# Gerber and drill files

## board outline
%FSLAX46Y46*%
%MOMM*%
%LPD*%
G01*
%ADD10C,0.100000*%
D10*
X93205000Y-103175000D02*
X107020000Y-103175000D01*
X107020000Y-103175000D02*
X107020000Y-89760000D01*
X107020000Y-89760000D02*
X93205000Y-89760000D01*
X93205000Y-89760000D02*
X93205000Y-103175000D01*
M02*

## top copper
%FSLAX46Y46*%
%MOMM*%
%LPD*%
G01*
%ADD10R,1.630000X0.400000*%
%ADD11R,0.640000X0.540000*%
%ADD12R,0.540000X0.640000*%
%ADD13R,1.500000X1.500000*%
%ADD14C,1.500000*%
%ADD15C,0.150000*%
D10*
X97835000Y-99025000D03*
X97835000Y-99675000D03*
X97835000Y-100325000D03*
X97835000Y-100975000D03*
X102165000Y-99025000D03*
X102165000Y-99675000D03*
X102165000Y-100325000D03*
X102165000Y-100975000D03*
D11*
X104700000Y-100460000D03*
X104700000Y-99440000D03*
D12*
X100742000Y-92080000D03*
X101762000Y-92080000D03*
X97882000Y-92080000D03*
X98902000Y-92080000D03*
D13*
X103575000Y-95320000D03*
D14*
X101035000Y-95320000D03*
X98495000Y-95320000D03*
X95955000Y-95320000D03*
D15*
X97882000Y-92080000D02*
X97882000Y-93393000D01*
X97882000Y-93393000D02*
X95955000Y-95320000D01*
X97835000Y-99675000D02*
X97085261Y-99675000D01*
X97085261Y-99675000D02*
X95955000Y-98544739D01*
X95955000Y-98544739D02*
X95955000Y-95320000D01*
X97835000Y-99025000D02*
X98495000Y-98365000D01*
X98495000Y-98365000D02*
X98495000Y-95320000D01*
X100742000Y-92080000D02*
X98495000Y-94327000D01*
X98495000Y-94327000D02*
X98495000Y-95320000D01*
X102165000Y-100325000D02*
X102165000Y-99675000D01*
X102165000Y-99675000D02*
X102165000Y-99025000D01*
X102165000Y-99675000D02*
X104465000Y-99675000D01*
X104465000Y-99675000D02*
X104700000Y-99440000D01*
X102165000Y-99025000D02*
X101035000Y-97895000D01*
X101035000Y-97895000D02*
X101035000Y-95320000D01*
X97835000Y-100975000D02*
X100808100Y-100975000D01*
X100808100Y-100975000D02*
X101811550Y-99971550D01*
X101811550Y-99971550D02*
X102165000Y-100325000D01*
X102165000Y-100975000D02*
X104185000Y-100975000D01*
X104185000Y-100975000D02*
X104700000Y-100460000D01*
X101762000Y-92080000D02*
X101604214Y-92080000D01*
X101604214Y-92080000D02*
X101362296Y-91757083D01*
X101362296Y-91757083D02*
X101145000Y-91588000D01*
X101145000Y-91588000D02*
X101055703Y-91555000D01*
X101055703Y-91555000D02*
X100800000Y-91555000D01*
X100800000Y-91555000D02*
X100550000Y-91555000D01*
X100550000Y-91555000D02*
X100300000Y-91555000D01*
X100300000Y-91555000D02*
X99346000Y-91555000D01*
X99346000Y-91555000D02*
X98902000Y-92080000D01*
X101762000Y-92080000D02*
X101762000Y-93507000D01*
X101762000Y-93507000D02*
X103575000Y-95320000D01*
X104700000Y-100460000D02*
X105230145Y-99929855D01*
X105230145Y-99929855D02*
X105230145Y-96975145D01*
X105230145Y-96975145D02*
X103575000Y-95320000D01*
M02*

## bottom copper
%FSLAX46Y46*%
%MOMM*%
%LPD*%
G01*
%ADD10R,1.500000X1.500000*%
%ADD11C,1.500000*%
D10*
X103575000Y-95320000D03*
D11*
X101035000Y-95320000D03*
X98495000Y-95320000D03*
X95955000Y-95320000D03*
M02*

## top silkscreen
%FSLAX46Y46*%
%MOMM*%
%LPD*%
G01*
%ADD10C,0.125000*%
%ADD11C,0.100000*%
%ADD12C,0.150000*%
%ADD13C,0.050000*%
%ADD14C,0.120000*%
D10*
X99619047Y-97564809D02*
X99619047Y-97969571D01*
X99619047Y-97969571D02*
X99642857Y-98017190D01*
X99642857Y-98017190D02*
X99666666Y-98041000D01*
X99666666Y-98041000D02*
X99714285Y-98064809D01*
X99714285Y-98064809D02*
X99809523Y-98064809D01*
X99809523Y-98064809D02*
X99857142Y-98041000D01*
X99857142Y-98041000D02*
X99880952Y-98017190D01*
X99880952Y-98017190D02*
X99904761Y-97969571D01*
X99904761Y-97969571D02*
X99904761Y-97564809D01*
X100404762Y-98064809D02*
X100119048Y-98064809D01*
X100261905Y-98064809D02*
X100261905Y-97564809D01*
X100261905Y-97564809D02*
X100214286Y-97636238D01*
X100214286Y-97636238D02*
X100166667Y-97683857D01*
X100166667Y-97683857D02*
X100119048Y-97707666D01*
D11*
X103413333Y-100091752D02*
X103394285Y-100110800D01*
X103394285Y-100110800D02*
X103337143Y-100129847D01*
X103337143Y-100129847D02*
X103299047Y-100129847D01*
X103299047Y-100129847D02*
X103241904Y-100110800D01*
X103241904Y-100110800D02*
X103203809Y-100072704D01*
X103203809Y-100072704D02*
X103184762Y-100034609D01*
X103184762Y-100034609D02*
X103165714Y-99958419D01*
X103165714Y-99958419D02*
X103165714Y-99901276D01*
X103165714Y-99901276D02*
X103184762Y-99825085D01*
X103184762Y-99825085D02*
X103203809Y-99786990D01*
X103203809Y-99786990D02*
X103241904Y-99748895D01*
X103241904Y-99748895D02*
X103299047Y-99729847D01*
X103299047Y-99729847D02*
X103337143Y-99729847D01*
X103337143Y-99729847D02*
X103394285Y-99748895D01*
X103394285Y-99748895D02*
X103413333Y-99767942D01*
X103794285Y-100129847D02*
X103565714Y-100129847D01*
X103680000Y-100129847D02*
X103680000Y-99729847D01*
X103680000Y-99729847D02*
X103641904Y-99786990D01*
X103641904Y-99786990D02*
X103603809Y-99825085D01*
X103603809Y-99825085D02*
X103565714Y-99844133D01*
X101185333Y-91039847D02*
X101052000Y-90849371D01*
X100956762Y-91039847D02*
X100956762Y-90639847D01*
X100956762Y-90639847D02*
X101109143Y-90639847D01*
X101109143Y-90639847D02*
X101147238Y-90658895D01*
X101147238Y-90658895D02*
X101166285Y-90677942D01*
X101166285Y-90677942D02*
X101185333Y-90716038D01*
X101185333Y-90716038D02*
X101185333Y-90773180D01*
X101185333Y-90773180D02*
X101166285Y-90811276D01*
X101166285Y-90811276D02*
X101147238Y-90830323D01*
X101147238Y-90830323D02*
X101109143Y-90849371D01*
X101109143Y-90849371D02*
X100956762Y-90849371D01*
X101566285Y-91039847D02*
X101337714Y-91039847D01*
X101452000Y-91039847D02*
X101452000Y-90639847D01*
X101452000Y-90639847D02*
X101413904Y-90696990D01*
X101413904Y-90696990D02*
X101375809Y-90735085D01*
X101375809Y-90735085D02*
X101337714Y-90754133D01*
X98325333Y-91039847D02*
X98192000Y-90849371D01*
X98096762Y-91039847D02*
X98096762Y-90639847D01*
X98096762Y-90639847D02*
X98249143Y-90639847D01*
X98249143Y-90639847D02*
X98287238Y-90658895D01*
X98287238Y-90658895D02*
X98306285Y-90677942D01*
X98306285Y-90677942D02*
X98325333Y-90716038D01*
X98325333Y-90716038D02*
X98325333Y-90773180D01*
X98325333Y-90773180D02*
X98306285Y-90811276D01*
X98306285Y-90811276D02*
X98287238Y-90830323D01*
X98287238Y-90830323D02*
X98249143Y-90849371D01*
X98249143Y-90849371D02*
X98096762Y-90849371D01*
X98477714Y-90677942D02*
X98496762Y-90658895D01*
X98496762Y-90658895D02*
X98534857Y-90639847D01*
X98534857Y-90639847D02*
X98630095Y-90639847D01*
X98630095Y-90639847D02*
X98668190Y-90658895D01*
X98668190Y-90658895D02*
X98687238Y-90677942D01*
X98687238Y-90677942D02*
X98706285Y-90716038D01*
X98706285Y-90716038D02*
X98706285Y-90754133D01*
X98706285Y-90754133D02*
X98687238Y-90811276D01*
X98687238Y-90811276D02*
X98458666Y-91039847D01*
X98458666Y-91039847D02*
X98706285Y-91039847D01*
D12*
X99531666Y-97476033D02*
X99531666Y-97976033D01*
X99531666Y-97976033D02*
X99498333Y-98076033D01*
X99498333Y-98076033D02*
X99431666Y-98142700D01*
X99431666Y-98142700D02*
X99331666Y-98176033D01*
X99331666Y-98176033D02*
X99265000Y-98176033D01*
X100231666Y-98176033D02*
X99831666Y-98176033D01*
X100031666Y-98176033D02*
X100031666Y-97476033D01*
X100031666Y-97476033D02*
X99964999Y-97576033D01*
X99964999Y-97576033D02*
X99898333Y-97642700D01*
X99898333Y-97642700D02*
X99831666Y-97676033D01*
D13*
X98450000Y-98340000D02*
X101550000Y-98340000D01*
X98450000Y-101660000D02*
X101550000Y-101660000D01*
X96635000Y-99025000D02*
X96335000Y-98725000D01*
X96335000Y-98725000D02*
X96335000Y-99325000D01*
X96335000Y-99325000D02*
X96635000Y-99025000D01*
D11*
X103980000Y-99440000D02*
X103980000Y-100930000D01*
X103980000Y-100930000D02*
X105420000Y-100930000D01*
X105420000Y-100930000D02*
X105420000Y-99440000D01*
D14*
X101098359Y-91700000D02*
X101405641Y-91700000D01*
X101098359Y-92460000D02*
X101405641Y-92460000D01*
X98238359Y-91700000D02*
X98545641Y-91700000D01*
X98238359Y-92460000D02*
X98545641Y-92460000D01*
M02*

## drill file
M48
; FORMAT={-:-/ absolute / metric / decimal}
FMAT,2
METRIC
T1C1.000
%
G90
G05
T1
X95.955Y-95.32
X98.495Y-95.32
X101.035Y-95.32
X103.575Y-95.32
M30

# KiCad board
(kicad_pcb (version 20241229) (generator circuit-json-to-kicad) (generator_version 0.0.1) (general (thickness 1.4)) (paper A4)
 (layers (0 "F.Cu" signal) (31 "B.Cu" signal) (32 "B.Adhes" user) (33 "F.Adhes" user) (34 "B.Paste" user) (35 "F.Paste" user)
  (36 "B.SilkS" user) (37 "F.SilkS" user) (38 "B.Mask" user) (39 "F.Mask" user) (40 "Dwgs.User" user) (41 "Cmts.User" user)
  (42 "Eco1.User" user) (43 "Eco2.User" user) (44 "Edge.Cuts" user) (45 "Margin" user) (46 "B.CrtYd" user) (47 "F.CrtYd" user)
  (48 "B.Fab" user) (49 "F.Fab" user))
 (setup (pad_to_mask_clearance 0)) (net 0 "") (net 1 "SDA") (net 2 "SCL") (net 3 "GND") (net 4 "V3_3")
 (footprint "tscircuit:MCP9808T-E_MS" (layer F.Cu) (at 100 100 0)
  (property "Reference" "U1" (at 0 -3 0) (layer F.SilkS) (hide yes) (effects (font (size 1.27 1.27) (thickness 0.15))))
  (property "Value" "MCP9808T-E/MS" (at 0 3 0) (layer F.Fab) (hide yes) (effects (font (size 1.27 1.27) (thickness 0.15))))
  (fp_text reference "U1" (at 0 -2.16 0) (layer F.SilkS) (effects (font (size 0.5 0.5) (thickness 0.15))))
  (fp_line (start -1.55 -1.66) (end 1.55 -1.66) (stroke (width 0.05) (type default)) (layer F.SilkS))
  (fp_line (start -1.55 1.66) (end 1.55 1.66) (stroke (width 0.05) (type default)) (layer F.SilkS))
  (fp_line (start -3.3649999999999998 -0.9750000000000001) (end -3.665 -1.2750000000000001) (stroke (width 0.05) (type default))
   (layer F.SilkS))
  (fp_line (start -3.665 -1.2750000000000001) (end -3.665 -0.675) (stroke (width 0.05) (type default)) (layer F.SilkS))
  (fp_line (start -3.665 -0.675) (end -3.3649999999999998 -0.9750000000000001) (stroke (width 0.05) (type default)) (layer F.SilkS))
  (pad "1" smd rect (at -2.165 -0.9750000000000001 0) (size 1.63 0.4) (layers F.Cu F.Paste F.Mask) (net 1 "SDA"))
  (pad "2" smd rect (at -2.165 -0.325 0) (size 1.63 0.4) (layers F.Cu F.Paste F.Mask) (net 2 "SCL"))
  (pad "3" smd rect (at -2.165 0.325 0) (size 1.63 0.4) (layers F.Cu F.Paste F.Mask))
  (pad "4" smd rect (at -2.165 0.9750000000000001 0) (size 1.63 0.4) (layers F.Cu F.Paste F.Mask) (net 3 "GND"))
  (pad "5" smd rect (at 2.165 -0.9750000000000001 0) (size 1.63 0.4) (layers F.Cu F.Paste F.Mask) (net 3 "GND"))
  (pad "6" smd rect (at 2.165 -0.325 0) (size 1.63 0.4) (layers F.Cu F.Paste F.Mask) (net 3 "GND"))
  (pad "7" smd rect (at 2.165 0.325 0) (size 1.63 0.4) (layers F.Cu F.Paste F.Mask) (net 3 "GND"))
  (pad "8" smd rect (at 2.165 0.9750000000000001 0) (size 1.63 0.4) (layers F.Cu F.Paste F.Mask) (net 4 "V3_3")))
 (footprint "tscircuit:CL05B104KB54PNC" (layer F.Cu) (at 104.7 99.95 90)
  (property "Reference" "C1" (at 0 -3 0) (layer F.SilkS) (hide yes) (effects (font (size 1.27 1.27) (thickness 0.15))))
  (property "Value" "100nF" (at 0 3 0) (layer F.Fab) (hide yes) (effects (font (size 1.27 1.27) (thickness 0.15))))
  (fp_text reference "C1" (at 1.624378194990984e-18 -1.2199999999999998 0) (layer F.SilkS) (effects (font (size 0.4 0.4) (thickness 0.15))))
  (fp_line (start 0.51 -0.7199999999999998) (end -0.98 -0.7200000000000001) (stroke (width 0.1) (type default)) (layer F.SilkS))
  (fp_line (start -0.98 -0.7200000000000001) (end -0.98 0.7199999999999999) (stroke (width 0.1) (type default)) (layer F.SilkS))
  (fp_line (start -0.98 0.7199999999999999) (end 0.51 0.7199999999999998) (stroke (width 0.1) (type default)) (layer F.SilkS))
  (pad "1" smd rect (at -0.51 0 0) (size 0.64 0.54) (layers F.Cu F.Paste F.Mask) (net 4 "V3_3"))
  (pad "2" smd rect (at 0.51 0 0) (size 0.64 0.54) (layers F.Cu F.Paste F.Mask) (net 3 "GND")))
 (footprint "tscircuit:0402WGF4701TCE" (layer F.Cu) (at 101.252 92.08 0)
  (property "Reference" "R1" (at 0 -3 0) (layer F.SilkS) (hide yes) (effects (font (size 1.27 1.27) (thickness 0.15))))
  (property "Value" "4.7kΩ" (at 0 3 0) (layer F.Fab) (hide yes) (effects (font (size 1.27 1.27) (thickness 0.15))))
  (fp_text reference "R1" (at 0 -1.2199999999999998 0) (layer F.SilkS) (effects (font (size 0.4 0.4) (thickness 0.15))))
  (fp_line (start -0.15364099999999992 -0.3799999999999999) (end 0.15364099999999992 -0.3799999999999999)
   (stroke (width 0.12) (type default)) (layer F.SilkS))
  (fp_line (start -0.15364099999999992 0.3799999999999999) (end 0.15364099999999992 0.3799999999999999) (stroke (width 0.12) (type default))
   (layer F.SilkS))
  (pad "1" smd rect (at -0.51 0 0) (size 0.54 0.64) (layers F.Cu F.Paste F.Mask) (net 1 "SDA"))
  (pad "2" smd rect (at 0.51 0 0) (size 0.54 0.64) (layers F.Cu F.Paste F.Mask) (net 4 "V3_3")))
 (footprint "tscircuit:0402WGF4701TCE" (layer F.Cu) (at 98.392 92.08 0)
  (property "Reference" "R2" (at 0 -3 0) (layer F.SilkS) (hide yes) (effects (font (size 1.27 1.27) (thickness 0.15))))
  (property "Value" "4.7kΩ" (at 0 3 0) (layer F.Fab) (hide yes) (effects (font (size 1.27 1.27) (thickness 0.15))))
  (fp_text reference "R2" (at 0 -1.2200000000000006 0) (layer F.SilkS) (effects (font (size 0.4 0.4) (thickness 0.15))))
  (fp_line (start -0.15364099999999992 -0.3800000000000008) (end 0.15364099999999992 -0.3800000000000008)
   (stroke (width 0.12) (type default)) (layer F.SilkS))
  (fp_line (start -0.15364099999999992 0.3799999999999999) (end 0.15364099999999992 0.3799999999999999) (stroke (width 0.12) (type default))
   (layer F.SilkS))
  (pad "1" smd rect (at -0.5099999999999998 0 0) (size 0.54 0.64) (layers F.Cu F.Paste F.Mask) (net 2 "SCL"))
  (pad "2" smd rect (at 0.51 0 0) (size 0.54 0.64) (layers F.Cu F.Paste F.Mask) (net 4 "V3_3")))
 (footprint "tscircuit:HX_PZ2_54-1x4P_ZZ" (layer F.Cu) (at 99.765 95.32 180)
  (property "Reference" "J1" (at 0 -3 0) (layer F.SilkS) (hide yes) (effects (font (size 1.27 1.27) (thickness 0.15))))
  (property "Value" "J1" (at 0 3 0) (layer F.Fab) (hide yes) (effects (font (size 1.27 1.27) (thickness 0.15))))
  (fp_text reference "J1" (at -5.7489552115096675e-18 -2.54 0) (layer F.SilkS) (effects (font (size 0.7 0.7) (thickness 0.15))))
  (pad "1" thru_hole rect (at -3.81 -4.215879892249837e-16 0) (size 1.5 1.5) (drill 1) (layers *.Cu *.Mask) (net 4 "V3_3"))
  (pad "2" thru_hole circle (at -1.27 1.5553014349171386e-16 0) (size 1.5 1.5) (drill 1) (layers *.Cu *.Mask) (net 3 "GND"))
  (pad "3" thru_hole circle (at 1.27 -1.5553014349171386e-16 0) (size 1.5 1.5) (drill 1) (layers *.Cu *.Mask) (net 1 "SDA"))
  (pad "4" thru_hole circle (at 3.8100000000000005 4.215879892249836e-16 0) (size 1.5 1.5) (drill 1) (layers *.Cu *.Mask) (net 2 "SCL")))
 (segment (start 97.882 92.08) (end 97.882 93.393) (width 0.15) (layer F.Cu) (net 2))
 (segment (start 97.882 93.393) (end 95.955 95.32) (width 0.15) (layer F.Cu) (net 2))
 (segment (start 97.835 99.675) (end 97.08526100782983 99.675) (width 0.15) (layer F.Cu) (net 2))
 (segment (start 97.08526100782983 99.675) (end 95.955 98.54473899217018) (width 0.15) (layer F.Cu) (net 2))
 (segment (start 95.955 98.54473899217018) (end 95.955 95.32) (width 0.15) (layer F.Cu) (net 2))
 (segment (start 97.835 99.025) (end 98.495 98.365) (width 0.15) (layer F.Cu) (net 1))
 (segment (start 98.495 98.365) (end 98.495 95.32) (width 0.15) (layer F.Cu) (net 1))
 (segment (start 100.742 92.08) (end 98.495 94.327) (width 0.15) (layer F.Cu) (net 1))
 (segment (start 98.495 94.327) (end 98.495 95.32) (width 0.15) (layer F.Cu) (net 1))
 (segment (start 102.165 100.325) (end 102.165 99.675) (width 0.15) (layer F.Cu) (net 3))
 (segment (start 102.165 99.675) (end 102.165 99.025) (width 0.15) (layer F.Cu) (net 3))
 (segment (start 102.165 99.675) (end 104.465 99.675) (width 0.15) (layer F.Cu) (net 3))
 (segment (start 104.465 99.675) (end 104.7 99.44) (width 0.15) (layer F.Cu) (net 3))
 (segment (start 102.165 99.025) (end 101.035 97.895) (width 0.15) (layer F.Cu) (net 3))
 (segment (start 101.035 97.895) (end 101.035 95.32) (width 0.15) (layer F.Cu) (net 3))
 (segment (start 97.835 100.975) (end 100.8081004428189 100.975) (width 0.15) (layer F.Cu) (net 3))
 (segment (start 100.8081004428189 100.975) (end 101.81155022140945 99.97155022140944) (width 0.15) (layer F.Cu) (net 3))
 (segment (start 101.81155022140945 99.97155022140944) (end 102.165 100.325) (width 0.15) (layer F.Cu) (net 3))
 (segment (start 102.165 100.975) (end 104.185 100.975) (width 0.15) (layer F.Cu) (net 4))
 (segment (start 104.185 100.975) (end 104.7 100.46) (width 0.15) (layer F.Cu) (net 4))
 (segment (start 101.762 92.08) (end 101.60421358827789 92.08) (width 0.15) (layer F.Cu) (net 4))
 (segment (start 101.60421358827789 92.08) (end 101.36229640972213 91.75708282144424) (width 0.15) (layer F.Cu) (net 4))
 (segment (start 101.36229640972213 91.75708282144424) (end 101.145 91.588) (width 0.15) (layer F.Cu) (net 4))
 (segment (start 101.145 91.588) (end 101.05570262747594 91.555) (width 0.15) (layer F.Cu) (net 4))
 (segment (start 101.05570262747594 91.555) (end 100.8 91.555) (width 0.15) (layer F.Cu) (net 4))
 (segment (start 100.8 91.555) (end 100.55 91.555) (width 0.15) (layer F.Cu) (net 4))
 (segment (start 100.55 91.555) (end 100.3 91.555) (width 0.15) (layer F.Cu) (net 4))
 (segment (start 100.3 91.555) (end 99.346 91.555) (width 0.15) (layer F.Cu) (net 4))
 (segment (start 99.346 91.555) (end 98.902 92.08) (width 0.15) (layer F.Cu) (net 4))
 (segment (start 101.762 92.08) (end 101.762 93.507) (width 0.15) (layer F.Cu) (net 4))
 (segment (start 101.762 93.507) (end 103.575 95.32) (width 0.15) (layer F.Cu) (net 4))
 (segment (start 104.7 100.46) (end 105.23014545291443 99.92985454708557) (width 0.15) (layer F.Cu) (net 4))
 (segment (start 105.23014545291443 99.92985454708557) (end 105.23014545291443 96.97514545291443) (width 0.15) (layer F.Cu) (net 4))
 (segment (start 105.23014545291443 96.97514545291443) (end 103.575 95.32) (width 0.15) (layer F.Cu) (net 4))
 (gr_line (start 93.205 103.175) (end 107.02 103.175) (width 0.1) (layer Edge.Cuts))
 (gr_line (start 107.02 103.175) (end 107.02 89.76) (width 0.1) (layer Edge.Cuts))
 (gr_line (start 107.02 89.76) (end 93.205 89.76) (width 0.1) (layer Edge.Cuts))
 (gr_line (start 93.205 89.76) (end 93.205 103.175) (width 0.1) (layer Edge.Cuts)))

